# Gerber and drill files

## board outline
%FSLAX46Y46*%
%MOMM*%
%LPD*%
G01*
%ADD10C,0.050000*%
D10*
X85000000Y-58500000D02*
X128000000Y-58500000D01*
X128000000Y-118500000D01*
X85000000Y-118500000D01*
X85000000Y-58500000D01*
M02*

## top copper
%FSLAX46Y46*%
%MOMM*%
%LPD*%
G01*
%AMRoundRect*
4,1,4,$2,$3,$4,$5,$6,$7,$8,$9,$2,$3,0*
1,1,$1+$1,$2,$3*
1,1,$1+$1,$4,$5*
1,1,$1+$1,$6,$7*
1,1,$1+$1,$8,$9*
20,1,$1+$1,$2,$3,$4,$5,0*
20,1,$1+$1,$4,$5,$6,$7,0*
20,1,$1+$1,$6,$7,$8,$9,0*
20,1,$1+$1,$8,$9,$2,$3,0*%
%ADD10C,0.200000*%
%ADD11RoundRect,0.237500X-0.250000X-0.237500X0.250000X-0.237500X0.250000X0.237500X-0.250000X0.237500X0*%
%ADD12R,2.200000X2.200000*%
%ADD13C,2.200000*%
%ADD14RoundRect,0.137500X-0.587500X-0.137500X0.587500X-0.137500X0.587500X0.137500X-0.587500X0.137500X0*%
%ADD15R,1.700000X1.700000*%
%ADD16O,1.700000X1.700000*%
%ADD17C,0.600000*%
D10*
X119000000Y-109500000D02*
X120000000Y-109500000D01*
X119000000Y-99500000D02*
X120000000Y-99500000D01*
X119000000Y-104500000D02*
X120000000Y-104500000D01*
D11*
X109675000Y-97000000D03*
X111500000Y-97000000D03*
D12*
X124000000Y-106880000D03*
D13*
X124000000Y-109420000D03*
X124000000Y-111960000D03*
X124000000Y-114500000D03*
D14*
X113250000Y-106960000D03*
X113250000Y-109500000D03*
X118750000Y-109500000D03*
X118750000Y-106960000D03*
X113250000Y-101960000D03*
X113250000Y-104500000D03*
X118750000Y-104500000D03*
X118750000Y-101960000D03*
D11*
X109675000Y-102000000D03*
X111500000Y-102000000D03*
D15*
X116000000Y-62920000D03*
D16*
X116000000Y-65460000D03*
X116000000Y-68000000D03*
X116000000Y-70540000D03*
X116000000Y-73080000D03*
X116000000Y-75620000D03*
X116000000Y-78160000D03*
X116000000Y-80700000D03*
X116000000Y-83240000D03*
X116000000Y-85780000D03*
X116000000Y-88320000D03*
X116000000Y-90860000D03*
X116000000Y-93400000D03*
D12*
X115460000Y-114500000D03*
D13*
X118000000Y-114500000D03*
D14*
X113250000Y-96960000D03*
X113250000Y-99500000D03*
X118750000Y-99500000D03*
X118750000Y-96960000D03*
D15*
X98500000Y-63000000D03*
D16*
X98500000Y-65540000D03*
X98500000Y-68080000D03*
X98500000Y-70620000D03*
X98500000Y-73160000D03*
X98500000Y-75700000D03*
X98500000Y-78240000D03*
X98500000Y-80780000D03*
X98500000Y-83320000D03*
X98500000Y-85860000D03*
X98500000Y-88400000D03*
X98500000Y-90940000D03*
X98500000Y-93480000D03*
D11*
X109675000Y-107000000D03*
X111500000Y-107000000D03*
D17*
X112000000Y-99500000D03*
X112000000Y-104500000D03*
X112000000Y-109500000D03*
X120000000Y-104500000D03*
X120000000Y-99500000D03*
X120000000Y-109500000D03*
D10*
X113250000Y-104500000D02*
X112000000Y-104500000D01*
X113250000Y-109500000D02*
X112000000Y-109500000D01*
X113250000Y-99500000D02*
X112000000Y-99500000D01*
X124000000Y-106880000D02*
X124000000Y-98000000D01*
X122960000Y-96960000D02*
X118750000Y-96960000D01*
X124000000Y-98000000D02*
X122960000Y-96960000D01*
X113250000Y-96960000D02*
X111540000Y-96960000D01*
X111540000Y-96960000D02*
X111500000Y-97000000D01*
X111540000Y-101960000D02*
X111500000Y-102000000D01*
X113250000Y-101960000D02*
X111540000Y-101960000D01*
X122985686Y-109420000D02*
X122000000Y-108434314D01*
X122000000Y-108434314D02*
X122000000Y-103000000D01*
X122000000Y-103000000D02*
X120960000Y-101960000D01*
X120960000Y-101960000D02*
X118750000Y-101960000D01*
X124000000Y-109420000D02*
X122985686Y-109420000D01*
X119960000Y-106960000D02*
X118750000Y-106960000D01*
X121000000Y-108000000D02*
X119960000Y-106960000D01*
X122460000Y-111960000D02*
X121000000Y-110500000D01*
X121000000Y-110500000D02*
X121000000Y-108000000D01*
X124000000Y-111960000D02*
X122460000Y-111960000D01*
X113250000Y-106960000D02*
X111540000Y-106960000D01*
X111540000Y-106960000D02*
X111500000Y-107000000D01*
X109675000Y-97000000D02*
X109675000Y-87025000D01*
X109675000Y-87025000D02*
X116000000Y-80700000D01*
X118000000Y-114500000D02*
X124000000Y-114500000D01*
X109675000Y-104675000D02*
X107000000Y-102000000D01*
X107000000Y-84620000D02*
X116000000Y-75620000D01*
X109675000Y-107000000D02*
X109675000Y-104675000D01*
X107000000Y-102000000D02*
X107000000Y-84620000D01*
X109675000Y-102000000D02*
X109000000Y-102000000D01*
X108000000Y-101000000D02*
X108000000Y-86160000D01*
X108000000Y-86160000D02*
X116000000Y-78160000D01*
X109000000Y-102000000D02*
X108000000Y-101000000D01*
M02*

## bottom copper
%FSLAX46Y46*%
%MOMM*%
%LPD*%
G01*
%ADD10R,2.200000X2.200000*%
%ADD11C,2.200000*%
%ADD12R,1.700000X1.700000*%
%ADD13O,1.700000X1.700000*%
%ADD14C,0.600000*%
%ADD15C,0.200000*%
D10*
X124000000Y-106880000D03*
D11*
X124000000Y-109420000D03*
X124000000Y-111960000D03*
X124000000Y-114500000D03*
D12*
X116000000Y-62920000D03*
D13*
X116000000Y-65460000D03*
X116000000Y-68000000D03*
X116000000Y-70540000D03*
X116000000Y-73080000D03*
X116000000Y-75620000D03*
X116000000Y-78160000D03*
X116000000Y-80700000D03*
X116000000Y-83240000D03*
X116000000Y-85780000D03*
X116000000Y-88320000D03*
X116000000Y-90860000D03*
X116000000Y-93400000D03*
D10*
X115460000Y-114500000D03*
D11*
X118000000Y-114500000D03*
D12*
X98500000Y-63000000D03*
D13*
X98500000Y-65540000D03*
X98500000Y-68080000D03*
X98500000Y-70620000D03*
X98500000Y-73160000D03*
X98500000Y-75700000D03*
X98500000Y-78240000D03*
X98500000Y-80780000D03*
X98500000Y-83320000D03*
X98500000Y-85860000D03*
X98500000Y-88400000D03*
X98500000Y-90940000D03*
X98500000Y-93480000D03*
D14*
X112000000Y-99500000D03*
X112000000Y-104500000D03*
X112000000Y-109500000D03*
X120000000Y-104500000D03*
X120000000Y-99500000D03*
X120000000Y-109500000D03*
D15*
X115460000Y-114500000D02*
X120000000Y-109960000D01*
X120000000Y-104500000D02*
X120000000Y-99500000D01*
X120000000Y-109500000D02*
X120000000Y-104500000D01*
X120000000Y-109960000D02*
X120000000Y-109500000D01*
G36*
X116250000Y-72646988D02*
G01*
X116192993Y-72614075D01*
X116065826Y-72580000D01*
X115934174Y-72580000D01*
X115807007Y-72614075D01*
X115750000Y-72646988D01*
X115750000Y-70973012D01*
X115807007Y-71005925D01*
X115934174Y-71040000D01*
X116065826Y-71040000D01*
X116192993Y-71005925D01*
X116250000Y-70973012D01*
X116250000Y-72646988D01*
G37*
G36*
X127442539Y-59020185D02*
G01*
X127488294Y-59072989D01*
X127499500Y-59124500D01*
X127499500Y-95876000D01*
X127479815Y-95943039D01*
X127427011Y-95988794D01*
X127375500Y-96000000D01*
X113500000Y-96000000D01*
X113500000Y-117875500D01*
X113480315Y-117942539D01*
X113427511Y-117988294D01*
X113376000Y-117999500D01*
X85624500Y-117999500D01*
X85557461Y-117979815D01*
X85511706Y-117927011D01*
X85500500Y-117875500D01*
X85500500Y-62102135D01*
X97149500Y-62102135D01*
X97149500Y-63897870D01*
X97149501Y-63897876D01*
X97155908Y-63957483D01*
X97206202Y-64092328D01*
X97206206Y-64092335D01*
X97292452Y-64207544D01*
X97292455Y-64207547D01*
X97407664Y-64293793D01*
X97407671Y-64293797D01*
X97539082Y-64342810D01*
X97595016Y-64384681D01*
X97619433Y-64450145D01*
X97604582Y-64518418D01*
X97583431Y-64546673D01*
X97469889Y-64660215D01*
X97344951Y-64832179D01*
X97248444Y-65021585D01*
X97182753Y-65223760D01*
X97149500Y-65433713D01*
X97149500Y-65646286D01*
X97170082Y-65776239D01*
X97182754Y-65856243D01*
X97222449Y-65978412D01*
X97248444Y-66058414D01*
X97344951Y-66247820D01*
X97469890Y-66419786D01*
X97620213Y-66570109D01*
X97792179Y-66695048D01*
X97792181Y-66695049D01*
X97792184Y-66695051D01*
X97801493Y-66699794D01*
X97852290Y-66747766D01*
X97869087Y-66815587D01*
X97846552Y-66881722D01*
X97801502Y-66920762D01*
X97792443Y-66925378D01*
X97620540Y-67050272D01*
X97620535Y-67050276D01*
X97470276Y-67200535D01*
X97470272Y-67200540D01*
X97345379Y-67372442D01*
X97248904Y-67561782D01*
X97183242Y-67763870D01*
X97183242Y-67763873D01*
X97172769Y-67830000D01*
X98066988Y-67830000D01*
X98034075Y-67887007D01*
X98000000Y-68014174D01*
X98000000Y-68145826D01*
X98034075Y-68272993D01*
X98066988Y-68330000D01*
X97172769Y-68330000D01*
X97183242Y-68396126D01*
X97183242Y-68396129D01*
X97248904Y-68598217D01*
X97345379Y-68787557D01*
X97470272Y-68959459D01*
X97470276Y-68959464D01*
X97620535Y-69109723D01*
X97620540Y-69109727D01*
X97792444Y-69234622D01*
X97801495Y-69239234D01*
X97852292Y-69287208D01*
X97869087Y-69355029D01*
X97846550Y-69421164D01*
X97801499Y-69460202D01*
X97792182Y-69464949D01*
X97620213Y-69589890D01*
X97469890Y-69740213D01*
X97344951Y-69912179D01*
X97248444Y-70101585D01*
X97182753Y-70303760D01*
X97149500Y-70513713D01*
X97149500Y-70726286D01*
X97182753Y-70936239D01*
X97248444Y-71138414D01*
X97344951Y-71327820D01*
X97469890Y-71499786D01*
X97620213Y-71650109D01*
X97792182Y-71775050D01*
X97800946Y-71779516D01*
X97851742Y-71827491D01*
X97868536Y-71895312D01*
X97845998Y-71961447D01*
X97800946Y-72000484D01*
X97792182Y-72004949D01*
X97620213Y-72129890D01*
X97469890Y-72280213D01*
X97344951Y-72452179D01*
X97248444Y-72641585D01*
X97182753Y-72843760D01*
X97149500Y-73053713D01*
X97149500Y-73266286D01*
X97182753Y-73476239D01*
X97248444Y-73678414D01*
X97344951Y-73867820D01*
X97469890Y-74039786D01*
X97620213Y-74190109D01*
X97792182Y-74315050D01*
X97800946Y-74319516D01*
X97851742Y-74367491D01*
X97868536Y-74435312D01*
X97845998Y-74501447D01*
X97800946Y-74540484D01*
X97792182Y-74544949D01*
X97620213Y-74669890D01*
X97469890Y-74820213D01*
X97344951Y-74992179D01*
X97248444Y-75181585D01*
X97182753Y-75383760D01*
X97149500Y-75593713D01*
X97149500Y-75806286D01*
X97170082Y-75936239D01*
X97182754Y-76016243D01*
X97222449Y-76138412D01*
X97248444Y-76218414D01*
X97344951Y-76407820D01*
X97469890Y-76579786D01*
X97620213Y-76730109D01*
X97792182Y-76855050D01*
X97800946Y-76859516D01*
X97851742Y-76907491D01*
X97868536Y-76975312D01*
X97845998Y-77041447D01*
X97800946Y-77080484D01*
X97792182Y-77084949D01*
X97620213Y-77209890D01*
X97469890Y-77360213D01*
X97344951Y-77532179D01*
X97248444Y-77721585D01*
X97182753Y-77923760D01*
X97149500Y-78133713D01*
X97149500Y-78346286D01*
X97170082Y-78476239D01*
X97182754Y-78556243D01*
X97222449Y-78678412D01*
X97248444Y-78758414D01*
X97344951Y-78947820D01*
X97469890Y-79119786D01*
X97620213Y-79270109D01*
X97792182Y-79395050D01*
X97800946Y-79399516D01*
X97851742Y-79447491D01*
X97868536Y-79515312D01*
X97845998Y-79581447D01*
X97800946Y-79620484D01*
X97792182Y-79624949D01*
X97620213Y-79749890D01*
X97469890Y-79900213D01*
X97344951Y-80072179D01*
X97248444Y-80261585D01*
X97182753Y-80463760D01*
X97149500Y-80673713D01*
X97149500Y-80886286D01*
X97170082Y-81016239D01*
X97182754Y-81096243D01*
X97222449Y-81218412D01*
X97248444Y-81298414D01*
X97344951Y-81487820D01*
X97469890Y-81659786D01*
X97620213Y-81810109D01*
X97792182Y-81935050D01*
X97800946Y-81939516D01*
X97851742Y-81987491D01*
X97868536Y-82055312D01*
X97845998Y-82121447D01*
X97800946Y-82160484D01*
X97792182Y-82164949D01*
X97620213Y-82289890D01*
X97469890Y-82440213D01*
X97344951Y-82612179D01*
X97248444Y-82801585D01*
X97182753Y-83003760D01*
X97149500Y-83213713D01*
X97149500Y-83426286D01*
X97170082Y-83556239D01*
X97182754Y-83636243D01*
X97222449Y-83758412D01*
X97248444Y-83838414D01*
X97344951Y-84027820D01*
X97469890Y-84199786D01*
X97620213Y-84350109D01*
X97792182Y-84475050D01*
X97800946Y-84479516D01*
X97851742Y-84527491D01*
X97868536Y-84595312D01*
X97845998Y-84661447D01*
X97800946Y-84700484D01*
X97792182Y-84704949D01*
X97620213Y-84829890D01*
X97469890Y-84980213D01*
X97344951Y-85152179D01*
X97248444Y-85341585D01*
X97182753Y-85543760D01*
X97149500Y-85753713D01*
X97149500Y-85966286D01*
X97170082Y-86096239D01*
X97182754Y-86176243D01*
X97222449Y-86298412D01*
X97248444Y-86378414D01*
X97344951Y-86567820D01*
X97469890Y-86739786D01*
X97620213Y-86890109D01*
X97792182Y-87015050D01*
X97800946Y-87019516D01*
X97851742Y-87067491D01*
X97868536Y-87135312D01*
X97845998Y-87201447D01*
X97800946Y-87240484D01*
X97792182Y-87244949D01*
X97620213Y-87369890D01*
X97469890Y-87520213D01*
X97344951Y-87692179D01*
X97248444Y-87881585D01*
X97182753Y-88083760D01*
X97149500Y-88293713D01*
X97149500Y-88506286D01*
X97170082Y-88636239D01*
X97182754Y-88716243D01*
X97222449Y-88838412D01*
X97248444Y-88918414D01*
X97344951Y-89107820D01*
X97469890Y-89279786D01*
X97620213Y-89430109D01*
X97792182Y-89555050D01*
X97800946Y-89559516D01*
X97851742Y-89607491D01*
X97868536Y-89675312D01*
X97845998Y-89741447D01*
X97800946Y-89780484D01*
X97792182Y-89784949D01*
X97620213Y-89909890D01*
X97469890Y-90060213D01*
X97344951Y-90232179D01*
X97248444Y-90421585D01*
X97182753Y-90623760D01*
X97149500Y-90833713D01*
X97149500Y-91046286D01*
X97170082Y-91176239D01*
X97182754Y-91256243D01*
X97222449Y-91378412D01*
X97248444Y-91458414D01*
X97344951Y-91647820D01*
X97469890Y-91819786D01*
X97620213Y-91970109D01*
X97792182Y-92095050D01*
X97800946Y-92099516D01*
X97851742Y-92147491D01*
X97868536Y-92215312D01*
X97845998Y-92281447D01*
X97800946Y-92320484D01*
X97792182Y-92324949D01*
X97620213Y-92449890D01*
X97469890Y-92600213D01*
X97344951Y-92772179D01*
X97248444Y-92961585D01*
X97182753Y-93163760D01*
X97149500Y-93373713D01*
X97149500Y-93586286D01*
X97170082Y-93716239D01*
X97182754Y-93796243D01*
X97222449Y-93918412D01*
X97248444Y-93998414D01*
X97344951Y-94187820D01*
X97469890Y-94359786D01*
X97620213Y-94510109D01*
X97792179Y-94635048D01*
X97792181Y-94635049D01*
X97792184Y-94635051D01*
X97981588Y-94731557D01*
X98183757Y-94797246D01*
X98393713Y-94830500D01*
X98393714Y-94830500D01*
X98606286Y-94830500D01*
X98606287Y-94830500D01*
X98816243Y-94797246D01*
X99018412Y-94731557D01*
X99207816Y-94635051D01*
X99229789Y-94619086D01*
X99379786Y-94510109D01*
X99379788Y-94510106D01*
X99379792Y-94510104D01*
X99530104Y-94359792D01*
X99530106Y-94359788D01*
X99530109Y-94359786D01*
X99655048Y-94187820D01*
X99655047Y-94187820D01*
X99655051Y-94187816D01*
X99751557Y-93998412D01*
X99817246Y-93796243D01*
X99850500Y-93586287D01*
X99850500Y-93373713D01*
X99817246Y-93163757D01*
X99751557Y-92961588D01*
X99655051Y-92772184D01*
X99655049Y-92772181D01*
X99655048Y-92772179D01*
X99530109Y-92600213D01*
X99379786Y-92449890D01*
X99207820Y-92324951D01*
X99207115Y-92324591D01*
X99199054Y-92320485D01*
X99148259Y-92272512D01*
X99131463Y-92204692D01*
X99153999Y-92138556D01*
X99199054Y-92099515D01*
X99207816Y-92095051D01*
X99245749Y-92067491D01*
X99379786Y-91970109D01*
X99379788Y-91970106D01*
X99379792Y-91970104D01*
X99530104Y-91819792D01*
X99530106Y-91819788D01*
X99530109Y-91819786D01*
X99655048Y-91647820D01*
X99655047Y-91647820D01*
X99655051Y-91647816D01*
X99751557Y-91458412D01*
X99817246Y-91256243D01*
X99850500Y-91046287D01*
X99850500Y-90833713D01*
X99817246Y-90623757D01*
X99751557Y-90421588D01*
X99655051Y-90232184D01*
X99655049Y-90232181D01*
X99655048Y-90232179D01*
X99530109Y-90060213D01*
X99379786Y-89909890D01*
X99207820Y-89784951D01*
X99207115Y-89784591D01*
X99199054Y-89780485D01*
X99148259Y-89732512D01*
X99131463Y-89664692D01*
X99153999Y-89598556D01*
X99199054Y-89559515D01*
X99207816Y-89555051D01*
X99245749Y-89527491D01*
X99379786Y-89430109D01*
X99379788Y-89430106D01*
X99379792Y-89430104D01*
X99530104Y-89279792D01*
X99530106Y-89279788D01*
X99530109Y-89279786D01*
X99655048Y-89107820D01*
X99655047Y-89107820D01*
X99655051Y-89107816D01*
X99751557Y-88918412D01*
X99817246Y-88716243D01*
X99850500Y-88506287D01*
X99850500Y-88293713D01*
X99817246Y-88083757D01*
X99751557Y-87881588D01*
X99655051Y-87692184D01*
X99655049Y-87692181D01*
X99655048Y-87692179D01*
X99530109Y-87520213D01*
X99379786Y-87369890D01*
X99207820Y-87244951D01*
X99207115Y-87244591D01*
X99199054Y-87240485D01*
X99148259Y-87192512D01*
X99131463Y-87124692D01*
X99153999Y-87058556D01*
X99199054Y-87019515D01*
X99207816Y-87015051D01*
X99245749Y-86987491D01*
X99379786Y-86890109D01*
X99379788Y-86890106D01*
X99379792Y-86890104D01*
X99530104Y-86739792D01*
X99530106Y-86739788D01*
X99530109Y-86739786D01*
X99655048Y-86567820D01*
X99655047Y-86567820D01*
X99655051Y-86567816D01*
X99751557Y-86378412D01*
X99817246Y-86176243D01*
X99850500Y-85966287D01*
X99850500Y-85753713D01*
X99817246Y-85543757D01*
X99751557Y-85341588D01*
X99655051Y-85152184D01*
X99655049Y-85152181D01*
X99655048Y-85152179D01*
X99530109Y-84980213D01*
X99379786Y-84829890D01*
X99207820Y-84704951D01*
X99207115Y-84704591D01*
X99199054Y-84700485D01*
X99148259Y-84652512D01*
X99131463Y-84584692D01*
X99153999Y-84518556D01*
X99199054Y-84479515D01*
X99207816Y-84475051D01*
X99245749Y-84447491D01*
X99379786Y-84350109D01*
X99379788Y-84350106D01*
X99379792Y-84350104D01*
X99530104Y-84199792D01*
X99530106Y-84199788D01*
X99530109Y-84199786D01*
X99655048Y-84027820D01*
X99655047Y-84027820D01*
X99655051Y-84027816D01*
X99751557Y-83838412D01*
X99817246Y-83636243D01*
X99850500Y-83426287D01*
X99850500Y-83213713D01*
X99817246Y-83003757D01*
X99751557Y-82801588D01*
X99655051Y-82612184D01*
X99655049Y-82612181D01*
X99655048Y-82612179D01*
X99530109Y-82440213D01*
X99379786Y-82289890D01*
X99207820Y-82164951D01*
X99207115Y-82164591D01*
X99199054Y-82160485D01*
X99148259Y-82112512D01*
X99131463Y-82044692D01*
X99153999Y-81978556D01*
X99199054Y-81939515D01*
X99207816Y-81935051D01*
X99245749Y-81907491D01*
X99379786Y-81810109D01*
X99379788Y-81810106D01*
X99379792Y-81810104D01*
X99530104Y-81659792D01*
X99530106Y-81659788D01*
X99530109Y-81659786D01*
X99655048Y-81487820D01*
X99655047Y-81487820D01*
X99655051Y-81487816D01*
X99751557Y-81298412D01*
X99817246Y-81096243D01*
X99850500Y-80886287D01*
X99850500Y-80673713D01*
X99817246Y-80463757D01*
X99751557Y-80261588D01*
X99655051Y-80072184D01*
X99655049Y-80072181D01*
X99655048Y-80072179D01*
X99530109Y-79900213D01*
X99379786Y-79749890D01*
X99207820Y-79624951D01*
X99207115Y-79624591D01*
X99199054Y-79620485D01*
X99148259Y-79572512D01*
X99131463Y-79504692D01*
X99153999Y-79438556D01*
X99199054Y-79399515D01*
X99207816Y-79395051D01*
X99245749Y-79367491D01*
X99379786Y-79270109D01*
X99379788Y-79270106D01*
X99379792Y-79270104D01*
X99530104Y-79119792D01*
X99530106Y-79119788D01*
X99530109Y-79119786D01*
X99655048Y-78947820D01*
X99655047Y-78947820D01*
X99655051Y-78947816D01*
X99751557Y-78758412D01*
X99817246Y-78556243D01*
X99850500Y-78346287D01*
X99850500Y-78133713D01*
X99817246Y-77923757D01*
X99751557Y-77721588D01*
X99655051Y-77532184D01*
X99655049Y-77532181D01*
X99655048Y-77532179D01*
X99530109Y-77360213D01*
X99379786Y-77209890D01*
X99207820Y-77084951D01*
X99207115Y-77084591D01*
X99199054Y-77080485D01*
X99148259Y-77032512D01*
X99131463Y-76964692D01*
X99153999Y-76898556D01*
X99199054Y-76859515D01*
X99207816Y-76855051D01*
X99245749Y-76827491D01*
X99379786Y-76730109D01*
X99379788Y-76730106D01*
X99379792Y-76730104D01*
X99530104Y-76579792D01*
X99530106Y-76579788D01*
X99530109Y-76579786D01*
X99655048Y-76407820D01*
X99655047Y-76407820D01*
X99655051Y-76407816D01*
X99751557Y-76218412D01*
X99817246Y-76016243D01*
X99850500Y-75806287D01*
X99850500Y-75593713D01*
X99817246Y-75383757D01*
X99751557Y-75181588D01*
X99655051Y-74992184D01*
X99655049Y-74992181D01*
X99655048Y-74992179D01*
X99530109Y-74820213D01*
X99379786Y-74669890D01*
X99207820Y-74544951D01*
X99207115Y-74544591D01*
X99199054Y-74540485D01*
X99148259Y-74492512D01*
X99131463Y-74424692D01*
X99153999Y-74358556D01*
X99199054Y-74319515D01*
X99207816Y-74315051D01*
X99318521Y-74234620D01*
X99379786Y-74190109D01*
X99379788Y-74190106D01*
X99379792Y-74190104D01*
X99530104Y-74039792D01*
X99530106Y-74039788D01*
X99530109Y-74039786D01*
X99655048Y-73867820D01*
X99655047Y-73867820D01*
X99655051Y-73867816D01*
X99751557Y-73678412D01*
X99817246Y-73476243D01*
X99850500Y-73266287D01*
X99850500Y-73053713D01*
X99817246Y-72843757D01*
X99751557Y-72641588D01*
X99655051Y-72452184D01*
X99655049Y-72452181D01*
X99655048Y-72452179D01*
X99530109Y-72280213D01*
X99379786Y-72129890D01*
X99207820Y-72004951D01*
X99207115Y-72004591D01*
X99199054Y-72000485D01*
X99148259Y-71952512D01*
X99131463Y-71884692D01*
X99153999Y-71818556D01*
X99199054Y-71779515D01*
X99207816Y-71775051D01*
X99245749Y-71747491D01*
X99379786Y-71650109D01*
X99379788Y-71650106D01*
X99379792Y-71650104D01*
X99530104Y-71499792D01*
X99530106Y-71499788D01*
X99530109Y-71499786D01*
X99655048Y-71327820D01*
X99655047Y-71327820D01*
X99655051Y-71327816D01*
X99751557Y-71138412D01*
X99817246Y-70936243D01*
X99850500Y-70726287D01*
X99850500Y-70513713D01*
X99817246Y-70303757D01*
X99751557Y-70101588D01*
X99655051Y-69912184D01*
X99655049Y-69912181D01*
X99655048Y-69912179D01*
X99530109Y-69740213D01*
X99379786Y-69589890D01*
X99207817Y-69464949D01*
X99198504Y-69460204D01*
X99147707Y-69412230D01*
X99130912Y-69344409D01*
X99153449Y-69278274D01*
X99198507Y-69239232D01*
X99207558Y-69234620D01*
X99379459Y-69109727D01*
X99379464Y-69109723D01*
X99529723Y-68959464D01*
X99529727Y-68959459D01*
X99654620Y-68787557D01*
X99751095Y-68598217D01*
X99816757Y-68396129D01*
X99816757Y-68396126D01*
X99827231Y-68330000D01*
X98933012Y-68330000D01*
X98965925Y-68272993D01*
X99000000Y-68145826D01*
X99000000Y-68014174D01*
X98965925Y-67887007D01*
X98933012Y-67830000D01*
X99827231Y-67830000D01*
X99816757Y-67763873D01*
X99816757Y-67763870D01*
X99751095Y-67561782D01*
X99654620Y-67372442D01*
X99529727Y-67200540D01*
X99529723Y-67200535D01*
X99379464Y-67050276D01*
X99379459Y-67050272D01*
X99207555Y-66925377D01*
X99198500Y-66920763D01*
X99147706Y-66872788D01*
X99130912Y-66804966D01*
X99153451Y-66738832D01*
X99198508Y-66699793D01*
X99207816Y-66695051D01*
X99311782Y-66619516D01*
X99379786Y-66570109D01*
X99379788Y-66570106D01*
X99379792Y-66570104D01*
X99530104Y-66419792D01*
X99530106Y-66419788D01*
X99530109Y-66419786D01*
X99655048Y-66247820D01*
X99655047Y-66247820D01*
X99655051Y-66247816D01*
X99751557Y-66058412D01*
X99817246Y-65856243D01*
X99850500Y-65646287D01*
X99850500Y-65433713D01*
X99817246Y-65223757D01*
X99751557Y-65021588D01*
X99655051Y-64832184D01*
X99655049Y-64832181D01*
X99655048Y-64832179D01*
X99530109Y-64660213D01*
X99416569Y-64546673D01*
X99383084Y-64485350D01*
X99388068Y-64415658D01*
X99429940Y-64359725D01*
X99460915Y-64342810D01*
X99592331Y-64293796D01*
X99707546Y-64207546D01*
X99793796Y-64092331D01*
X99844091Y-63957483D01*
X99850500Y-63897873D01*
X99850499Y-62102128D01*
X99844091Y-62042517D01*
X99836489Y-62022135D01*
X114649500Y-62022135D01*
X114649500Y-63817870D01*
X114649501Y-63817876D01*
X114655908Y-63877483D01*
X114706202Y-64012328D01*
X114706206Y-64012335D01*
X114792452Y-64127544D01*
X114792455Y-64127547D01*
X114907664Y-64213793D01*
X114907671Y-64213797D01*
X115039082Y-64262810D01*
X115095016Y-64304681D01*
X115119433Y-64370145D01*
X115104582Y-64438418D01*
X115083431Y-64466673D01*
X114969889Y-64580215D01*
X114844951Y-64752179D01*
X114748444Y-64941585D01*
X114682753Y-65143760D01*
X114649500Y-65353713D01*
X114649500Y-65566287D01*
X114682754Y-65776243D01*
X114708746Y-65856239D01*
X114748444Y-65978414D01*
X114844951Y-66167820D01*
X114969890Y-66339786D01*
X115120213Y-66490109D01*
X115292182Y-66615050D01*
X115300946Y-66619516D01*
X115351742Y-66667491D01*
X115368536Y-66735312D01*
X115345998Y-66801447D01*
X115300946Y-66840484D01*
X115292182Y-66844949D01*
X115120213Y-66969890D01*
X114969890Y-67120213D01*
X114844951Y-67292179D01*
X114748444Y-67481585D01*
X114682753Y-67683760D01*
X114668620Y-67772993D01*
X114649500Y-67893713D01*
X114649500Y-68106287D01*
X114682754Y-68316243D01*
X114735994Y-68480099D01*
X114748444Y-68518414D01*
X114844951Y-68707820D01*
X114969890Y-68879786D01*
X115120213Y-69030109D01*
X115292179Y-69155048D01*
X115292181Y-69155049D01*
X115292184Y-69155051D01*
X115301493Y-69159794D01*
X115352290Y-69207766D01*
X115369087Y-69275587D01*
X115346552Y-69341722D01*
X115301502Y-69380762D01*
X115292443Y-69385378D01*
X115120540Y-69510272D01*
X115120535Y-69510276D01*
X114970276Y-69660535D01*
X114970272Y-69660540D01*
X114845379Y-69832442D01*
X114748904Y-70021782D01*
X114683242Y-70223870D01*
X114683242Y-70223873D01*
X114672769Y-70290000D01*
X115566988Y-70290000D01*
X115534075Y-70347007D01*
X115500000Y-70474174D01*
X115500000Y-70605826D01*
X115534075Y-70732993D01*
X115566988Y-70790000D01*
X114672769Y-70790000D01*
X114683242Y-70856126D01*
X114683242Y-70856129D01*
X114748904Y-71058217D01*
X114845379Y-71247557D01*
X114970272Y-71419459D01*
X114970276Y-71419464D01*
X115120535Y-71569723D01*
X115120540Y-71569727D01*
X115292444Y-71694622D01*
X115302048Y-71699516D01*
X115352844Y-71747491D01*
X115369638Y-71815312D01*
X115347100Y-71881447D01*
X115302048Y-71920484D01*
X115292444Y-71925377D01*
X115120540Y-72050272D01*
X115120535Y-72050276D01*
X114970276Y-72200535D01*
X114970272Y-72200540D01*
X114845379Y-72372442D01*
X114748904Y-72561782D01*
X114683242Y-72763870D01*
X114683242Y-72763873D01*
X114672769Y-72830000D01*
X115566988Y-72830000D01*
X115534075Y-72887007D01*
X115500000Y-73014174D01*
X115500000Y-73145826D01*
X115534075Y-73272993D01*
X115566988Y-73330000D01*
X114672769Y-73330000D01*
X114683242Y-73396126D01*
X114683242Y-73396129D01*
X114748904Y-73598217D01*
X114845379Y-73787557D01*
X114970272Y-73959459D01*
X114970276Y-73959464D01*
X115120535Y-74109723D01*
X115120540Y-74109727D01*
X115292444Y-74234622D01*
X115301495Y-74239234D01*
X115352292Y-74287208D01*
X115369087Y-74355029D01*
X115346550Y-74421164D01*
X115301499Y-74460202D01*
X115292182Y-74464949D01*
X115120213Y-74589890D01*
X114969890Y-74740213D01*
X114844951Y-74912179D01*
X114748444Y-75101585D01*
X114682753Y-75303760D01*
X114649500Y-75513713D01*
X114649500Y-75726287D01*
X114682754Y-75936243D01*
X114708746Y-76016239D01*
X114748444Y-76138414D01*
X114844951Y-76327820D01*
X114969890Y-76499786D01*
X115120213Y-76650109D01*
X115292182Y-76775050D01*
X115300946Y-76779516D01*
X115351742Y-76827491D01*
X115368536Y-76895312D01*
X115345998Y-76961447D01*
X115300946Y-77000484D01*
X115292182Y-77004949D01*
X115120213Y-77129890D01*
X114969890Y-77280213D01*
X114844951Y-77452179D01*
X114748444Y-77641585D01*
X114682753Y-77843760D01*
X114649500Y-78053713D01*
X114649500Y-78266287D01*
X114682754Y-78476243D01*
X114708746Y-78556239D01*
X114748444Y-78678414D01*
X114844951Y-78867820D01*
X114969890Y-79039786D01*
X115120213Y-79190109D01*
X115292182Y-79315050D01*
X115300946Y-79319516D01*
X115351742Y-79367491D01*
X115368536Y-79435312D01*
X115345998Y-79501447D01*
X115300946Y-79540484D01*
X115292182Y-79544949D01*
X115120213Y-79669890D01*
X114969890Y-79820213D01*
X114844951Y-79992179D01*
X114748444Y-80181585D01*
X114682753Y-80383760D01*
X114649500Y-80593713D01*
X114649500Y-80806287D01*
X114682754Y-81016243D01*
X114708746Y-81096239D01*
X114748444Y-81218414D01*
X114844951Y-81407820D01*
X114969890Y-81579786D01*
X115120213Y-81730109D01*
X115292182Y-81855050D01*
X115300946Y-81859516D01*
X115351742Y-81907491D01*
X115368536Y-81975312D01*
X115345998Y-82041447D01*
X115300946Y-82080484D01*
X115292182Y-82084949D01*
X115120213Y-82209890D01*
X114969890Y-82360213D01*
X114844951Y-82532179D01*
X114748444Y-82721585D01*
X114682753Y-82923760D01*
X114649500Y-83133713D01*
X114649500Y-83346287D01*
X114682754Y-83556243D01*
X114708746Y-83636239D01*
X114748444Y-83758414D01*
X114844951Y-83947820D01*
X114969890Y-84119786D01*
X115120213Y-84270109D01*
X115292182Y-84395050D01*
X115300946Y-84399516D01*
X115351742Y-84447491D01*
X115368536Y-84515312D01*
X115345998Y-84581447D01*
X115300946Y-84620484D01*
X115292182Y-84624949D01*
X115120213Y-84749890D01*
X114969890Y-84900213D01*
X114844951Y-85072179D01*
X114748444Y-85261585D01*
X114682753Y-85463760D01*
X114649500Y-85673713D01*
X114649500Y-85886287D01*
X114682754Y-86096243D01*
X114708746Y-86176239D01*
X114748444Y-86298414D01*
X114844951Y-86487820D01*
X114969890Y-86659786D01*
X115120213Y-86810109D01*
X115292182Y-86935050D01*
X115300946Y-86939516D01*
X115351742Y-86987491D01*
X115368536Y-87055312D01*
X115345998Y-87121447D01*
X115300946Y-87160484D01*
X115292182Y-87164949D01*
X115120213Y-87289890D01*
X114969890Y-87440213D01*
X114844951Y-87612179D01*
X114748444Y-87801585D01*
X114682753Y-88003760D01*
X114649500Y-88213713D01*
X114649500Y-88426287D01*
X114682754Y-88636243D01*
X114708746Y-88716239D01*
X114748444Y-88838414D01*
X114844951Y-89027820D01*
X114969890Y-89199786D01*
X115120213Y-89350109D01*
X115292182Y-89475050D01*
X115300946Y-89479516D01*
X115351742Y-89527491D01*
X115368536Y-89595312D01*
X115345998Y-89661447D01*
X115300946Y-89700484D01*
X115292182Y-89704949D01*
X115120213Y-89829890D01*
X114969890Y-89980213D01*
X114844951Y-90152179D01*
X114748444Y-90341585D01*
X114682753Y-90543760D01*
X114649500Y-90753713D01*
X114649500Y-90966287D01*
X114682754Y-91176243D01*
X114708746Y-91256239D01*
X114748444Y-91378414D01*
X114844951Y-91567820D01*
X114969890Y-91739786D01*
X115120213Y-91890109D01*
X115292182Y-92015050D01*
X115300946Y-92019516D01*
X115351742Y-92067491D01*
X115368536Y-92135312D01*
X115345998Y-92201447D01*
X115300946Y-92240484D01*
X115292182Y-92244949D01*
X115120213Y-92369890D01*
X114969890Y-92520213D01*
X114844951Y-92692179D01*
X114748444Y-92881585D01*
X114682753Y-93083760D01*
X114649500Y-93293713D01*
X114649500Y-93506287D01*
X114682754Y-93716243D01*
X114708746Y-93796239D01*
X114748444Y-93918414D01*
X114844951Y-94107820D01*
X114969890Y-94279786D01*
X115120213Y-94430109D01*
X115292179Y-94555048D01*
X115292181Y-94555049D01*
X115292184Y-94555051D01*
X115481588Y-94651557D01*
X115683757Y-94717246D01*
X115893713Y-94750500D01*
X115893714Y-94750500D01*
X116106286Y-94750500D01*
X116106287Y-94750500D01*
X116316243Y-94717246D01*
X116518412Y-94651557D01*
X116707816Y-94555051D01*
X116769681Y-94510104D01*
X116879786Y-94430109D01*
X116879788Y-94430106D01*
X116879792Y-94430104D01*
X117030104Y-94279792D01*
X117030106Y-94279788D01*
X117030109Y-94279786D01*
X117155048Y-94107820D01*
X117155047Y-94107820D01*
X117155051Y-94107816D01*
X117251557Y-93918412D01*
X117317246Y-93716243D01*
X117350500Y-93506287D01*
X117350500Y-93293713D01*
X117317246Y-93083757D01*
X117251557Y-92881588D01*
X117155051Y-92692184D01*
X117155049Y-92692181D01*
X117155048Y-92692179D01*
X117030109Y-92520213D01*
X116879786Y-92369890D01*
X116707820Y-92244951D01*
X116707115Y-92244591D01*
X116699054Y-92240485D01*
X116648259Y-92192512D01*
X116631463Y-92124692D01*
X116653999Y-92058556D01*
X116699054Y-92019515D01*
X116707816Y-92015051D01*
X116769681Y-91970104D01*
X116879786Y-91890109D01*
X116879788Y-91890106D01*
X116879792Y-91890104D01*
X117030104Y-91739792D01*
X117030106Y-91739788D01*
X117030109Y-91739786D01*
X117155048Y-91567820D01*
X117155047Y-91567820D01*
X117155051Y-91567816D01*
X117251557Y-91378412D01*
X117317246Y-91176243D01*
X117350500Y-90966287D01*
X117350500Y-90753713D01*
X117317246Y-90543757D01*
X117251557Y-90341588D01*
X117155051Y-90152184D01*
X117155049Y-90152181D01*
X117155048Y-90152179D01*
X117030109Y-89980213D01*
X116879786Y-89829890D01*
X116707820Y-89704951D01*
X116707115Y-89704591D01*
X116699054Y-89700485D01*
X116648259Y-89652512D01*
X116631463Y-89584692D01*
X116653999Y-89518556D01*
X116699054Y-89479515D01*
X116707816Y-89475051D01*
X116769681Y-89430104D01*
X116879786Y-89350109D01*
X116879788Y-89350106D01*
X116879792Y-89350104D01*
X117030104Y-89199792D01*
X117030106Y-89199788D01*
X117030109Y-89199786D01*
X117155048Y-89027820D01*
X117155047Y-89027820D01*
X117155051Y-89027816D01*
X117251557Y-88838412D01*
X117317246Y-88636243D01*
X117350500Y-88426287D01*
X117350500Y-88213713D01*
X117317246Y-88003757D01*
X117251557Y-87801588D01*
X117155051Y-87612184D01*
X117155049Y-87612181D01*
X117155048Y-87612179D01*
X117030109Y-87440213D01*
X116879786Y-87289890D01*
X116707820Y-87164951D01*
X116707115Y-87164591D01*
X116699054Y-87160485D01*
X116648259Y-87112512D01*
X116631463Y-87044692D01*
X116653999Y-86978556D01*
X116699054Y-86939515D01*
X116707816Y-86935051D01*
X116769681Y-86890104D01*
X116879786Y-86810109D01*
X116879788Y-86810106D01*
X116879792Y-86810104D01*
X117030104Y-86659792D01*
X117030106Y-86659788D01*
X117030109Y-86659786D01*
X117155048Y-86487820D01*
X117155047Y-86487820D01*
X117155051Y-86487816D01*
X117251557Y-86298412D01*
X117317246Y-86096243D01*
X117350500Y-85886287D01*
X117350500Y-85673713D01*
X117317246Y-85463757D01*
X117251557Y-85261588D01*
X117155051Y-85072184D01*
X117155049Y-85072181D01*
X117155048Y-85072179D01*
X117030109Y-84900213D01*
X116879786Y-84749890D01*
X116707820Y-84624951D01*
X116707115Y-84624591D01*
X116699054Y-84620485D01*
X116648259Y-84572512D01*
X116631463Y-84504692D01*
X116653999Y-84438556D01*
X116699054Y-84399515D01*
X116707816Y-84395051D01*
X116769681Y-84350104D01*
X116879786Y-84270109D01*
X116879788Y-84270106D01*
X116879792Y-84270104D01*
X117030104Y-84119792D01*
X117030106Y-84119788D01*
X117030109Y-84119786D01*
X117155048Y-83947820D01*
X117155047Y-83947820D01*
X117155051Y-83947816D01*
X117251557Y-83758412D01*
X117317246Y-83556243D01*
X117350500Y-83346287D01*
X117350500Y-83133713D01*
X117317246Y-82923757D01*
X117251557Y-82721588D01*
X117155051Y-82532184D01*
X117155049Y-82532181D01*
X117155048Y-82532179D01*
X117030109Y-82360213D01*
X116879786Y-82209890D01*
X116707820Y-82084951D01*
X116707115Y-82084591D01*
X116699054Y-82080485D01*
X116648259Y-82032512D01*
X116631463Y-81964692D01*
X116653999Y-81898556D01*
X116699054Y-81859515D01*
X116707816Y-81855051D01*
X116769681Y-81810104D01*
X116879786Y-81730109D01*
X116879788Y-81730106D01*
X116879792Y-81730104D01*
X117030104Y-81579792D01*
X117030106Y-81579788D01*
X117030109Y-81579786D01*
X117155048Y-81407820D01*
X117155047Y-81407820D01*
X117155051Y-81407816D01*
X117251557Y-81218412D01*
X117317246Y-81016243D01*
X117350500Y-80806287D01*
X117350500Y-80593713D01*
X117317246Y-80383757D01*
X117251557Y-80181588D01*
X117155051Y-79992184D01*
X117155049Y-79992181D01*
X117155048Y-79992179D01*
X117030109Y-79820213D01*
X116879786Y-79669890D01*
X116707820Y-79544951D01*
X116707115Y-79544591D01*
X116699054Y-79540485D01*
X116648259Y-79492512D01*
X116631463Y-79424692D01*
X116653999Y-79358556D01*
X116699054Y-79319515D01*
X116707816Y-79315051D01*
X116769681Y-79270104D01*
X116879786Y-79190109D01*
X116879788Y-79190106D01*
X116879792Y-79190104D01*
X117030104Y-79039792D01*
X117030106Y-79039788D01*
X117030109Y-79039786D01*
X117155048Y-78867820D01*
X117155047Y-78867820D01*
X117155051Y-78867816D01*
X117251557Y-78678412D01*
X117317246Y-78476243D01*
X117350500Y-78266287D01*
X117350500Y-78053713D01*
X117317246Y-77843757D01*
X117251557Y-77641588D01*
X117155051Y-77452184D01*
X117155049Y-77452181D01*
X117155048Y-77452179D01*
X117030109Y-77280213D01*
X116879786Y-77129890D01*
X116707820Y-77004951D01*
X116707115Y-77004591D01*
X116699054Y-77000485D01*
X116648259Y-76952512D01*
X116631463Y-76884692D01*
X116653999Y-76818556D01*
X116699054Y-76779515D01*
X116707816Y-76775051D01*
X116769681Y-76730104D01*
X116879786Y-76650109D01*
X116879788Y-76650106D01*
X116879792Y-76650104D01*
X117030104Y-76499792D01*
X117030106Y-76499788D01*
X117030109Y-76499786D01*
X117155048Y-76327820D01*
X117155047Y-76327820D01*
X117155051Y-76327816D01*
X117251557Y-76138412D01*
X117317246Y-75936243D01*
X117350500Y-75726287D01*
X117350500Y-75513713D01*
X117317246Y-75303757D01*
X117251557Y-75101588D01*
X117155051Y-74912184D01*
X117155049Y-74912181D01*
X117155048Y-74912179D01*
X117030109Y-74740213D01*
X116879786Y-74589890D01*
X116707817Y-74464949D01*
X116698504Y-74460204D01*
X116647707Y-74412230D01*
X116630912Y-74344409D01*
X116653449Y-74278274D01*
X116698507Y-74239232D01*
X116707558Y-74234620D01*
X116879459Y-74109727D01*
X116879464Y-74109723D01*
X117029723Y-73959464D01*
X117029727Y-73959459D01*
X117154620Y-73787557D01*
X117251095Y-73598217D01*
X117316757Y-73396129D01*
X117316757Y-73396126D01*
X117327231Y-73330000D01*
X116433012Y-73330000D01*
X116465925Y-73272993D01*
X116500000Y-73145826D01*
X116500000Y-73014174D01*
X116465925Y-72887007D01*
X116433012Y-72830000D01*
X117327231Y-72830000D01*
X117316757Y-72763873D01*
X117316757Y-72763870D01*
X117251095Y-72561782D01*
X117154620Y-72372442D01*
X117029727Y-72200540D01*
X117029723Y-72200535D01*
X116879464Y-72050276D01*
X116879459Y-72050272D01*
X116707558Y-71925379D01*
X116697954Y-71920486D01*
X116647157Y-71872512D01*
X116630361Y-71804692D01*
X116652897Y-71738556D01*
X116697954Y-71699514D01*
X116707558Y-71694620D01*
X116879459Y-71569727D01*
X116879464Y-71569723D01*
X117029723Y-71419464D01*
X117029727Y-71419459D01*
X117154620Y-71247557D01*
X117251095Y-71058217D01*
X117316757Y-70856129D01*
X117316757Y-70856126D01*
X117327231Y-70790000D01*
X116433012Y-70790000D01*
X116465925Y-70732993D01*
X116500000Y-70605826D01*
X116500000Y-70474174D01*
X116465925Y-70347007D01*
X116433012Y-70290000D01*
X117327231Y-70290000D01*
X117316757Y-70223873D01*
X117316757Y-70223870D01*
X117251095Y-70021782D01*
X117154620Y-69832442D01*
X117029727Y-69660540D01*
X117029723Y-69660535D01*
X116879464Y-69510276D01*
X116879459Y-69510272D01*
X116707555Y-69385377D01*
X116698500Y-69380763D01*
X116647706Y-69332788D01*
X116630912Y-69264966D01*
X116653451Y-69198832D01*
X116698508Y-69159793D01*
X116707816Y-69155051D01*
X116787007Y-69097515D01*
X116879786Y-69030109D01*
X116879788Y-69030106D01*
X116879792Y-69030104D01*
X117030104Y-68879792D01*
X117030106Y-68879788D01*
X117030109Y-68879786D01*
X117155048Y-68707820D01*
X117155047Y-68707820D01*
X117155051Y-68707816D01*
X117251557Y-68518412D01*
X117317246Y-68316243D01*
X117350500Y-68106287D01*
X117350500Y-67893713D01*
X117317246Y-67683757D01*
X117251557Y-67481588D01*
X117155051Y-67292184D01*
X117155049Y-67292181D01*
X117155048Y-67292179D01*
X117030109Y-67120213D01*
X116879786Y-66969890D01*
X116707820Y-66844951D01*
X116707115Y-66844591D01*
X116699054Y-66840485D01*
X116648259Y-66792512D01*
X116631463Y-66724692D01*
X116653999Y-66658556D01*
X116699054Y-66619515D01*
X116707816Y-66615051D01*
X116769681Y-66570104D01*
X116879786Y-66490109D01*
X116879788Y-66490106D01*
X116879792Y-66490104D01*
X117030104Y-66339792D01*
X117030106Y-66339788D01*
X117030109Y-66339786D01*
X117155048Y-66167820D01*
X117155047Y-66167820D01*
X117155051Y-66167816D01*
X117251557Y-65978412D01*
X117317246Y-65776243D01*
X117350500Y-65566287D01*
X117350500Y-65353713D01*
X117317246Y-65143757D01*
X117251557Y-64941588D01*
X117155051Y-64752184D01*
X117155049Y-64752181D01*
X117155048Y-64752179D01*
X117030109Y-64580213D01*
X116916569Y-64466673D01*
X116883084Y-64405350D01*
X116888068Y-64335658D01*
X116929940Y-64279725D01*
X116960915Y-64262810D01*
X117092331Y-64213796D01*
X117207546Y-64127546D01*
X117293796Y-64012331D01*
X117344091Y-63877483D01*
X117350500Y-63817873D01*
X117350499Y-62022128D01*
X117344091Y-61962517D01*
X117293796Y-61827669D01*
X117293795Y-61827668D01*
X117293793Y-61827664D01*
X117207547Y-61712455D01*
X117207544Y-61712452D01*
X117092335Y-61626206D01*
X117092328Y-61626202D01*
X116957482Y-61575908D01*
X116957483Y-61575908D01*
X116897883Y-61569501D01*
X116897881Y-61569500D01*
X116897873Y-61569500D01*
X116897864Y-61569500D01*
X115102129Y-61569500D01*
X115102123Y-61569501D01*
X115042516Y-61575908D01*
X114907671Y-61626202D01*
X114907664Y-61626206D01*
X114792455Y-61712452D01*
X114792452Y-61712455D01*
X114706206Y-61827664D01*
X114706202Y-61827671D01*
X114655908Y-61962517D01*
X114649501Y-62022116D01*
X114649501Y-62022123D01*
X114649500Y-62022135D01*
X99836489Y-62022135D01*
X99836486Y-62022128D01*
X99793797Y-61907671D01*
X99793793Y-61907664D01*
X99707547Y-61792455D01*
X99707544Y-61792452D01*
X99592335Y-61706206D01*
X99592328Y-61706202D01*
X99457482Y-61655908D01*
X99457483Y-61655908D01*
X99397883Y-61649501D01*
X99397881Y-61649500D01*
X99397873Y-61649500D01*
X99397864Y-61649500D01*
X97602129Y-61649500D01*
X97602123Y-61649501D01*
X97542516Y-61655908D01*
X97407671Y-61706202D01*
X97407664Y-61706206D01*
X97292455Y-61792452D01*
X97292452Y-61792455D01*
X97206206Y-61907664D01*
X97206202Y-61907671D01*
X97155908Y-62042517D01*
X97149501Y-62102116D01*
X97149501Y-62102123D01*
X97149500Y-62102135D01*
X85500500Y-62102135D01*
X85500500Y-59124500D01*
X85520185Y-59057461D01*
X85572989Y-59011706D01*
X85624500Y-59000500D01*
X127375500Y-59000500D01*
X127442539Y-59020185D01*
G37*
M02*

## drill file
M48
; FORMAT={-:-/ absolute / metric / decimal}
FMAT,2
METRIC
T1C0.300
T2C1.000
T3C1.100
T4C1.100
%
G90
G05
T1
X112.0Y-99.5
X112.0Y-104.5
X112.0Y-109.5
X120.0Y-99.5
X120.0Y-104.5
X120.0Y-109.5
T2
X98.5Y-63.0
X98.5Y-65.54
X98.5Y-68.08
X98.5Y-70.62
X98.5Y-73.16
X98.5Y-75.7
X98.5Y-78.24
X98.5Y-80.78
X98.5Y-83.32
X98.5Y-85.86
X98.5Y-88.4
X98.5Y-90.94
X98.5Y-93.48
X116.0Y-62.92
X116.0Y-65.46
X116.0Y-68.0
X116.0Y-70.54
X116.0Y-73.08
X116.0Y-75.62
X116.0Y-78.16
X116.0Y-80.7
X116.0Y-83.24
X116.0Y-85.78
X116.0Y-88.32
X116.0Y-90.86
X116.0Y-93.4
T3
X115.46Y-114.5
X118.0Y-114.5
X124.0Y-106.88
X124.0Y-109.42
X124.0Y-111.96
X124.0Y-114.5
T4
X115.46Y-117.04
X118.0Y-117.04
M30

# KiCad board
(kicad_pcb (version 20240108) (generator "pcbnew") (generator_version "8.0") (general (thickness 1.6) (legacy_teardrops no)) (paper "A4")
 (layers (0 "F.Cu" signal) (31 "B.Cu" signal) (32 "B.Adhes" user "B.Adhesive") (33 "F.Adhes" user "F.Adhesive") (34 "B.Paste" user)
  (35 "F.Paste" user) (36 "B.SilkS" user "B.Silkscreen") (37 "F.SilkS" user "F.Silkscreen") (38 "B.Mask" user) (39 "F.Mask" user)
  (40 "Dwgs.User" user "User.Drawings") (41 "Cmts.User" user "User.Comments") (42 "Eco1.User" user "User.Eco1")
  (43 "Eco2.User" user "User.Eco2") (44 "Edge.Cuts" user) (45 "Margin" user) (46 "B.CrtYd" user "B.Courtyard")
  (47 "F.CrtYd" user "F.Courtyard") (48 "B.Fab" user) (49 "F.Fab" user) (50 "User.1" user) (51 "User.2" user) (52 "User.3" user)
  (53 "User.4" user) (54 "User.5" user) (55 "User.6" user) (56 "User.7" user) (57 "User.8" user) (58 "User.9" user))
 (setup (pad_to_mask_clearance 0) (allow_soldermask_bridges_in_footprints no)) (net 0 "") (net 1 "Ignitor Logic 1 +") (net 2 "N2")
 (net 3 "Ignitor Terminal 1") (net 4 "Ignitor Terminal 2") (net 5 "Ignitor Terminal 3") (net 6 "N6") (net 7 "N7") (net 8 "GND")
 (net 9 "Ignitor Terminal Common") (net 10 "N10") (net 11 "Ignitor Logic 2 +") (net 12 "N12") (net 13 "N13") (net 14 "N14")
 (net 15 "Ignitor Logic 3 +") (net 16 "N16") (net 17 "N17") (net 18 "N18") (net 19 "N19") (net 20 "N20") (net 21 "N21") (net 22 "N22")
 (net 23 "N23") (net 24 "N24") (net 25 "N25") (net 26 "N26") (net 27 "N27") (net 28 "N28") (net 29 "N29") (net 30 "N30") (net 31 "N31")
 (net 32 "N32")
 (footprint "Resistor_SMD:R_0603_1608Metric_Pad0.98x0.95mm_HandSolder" (layer "F.Cu") (at 110.5875 97)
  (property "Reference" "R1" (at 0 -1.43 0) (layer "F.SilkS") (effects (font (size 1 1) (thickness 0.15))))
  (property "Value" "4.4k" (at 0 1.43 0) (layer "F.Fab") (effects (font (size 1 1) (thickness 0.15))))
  (pad "1" smd roundrect (at -0.9125 0) (size 0.975 0.95) (layers "F.Cu" "F.Paste" "F.Mask") (roundrect_rratio 0.25)
   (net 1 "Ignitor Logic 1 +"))
  (pad "2" smd roundrect (at 0.9125 0) (size 0.975 0.95) (layers "F.Cu" "F.Paste" "F.Mask") (roundrect_rratio 0.25) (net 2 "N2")))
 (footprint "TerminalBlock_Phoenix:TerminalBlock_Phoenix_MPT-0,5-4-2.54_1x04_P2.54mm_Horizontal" (layer "F.Cu") (at 124 106.88 -90)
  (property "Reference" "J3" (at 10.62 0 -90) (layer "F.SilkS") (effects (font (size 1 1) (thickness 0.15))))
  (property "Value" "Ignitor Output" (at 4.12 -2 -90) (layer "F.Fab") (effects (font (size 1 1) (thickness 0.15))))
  (pad "1" thru_hole rect (at 0 0 270) (size 2.2 2.2) (drill 1.1) (layers "*.Cu" "*.Mask") (remove_unused_layers no)
   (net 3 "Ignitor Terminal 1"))
  (pad "2" thru_hole circle (at 2.54 0 270) (size 2.2 2.2) (drill 1.1) (layers "*.Cu" "*.Mask") (remove_unused_layers no)
   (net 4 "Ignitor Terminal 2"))
  (pad "3" thru_hole circle (at 5.08 0 270) (size 2.2 2.2) (drill 1.1) (layers "*.Cu" "*.Mask") (remove_unused_layers no)
   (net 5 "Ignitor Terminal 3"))
  (pad "4" thru_hole circle (at 7.62 0 270) (size 2.2 2.2) (drill 1.1) (layers "*.Cu" "*.Mask") (remove_unused_layers no) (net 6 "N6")))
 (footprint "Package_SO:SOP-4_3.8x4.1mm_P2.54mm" (layer "F.Cu") (at 116 108.23)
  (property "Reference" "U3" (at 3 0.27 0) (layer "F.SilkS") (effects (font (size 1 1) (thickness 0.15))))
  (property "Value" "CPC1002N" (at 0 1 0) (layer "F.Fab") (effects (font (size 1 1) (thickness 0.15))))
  (pad "1" smd roundrect (at -2.75 -1.27) (size 1.45 0.55) (layers "F.Cu" "F.Paste" "F.Mask") (roundrect_rratio 0.25) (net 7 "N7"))
  (pad "2" smd roundrect (at -2.75 1.27) (size 1.45 0.55) (layers "F.Cu" "F.Paste" "F.Mask") (roundrect_rratio 0.25) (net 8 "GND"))
  (pad "3" smd roundrect (at 2.75 1.27) (size 1.45 0.55) (layers "F.Cu" "F.Paste" "F.Mask") (roundrect_rratio 0.25)
   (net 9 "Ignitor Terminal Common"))
  (pad "4" smd roundrect (at 2.75 -1.27) (size 1.45 0.55) (layers "F.Cu" "F.Paste" "F.Mask") (roundrect_rratio 0.25)
   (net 5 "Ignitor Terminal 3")))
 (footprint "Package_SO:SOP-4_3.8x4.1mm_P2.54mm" (layer "F.Cu") (at 116 103.23)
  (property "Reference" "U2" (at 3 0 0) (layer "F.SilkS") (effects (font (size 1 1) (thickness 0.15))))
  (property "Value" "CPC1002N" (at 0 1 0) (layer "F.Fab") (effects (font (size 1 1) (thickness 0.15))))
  (pad "1" smd roundrect (at -2.75 -1.27) (size 1.45 0.55) (layers "F.Cu" "F.Paste" "F.Mask") (roundrect_rratio 0.25) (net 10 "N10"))
  (pad "2" smd roundrect (at -2.75 1.27) (size 1.45 0.55) (layers "F.Cu" "F.Paste" "F.Mask") (roundrect_rratio 0.25) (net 8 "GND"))
  (pad "3" smd roundrect (at 2.75 1.27) (size 1.45 0.55) (layers "F.Cu" "F.Paste" "F.Mask") (roundrect_rratio 0.25)
   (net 9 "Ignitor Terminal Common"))
  (pad "4" smd roundrect (at 2.75 -1.27) (size 1.45 0.55) (layers "F.Cu" "F.Paste" "F.Mask") (roundrect_rratio 0.25)
   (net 4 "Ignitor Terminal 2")))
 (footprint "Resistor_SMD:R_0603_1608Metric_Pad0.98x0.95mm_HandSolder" (layer "F.Cu") (at 110.5875 102)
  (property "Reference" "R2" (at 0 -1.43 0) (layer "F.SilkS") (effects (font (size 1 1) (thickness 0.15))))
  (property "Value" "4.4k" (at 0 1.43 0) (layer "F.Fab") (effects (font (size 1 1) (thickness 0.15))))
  (pad "1" smd roundrect (at -0.9125 0) (size 0.975 0.95) (layers "F.Cu" "F.Paste" "F.Mask") (roundrect_rratio 0.25)
   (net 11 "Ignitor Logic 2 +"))
  (pad "2" smd roundrect (at 0.9125 0) (size 0.975 0.95) (layers "F.Cu" "F.Paste" "F.Mask") (roundrect_rratio 0.25) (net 10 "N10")))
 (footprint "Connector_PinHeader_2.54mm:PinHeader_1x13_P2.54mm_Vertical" (layer "F.Cu") (at 116 62.92)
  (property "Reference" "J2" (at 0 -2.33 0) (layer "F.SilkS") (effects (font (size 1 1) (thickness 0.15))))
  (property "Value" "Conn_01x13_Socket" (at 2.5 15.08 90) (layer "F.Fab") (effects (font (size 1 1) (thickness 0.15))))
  (pad "1" thru_hole rect (at 0 0) (size 1.7 1.7) (drill 1) (layers "*.Cu" "*.Mask") (remove_unused_layers no) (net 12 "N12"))
  (pad "2" thru_hole oval (at 0 2.54) (size 1.7 1.7) (drill 1) (layers "*.Cu" "*.Mask") (remove_unused_layers no) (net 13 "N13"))
  (pad "3" thru_hole oval (at 0 5.08) (size 1.7 1.7) (drill 1) (layers "*.Cu" "*.Mask") (remove_unused_layers no) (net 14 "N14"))
  (pad "4" thru_hole oval (at 0 7.62) (size 1.7 1.7) (drill 1) (layers "*.Cu" "*.Mask") (remove_unused_layers no) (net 8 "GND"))
  (pad "5" thru_hole oval (at 0 10.16) (size 1.7 1.7) (drill 1) (layers "*.Cu" "*.Mask") (remove_unused_layers no) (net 8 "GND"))
  (pad "6" thru_hole oval (at 0 12.7) (size 1.7 1.7) (drill 1) (layers "*.Cu" "*.Mask") (remove_unused_layers no)
   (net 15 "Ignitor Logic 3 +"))
  (pad "7" thru_hole oval (at 0 15.24) (size 1.7 1.7) (drill 1) (layers "*.Cu" "*.Mask") (remove_unused_layers no)
   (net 11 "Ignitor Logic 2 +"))
  (pad "8" thru_hole oval (at 0 17.78) (size 1.7 1.7) (drill 1) (layers "*.Cu" "*.Mask") (remove_unused_layers no)
   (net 1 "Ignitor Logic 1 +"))
  (pad "9" thru_hole oval (at 0 20.32) (size 1.7 1.7) (drill 1) (layers "*.Cu" "*.Mask") (remove_unused_layers no) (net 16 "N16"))
  (pad "10" thru_hole oval (at 0 22.86) (size 1.7 1.7) (drill 1) (layers "*.Cu" "*.Mask") (remove_unused_layers no) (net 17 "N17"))
  (pad "11" thru_hole oval (at 0 25.4) (size 1.7 1.7) (drill 1) (layers "*.Cu" "*.Mask") (remove_unused_layers no) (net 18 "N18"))
  (pad "12" thru_hole oval (at 0 27.94) (size 1.7 1.7) (drill 1) (layers "*.Cu" "*.Mask") (remove_unused_layers no) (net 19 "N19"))
  (pad "13" thru_hole oval (at 0 30.48) (size 1.7 1.7) (drill 1) (layers "*.Cu" "*.Mask") (remove_unused_layers no) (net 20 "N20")))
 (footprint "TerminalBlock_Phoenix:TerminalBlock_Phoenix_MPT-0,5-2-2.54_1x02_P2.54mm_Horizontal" (layer "F.Cu") (at 115.46 114.5)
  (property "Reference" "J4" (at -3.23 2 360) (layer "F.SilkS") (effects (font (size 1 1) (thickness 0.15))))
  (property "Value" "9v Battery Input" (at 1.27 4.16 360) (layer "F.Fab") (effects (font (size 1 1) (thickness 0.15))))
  (pad "" np_thru_hole circle (at 0 2.54) (size 1.1 1.1) (drill 1.1) (layers "*.Cu" "*.Mask"))
  (pad "" np_thru_hole circle (at 2.54 2.54) (size 1.1 1.1) (drill 1.1) (layers "*.Cu" "*.Mask"))
  (pad "1" thru_hole rect (at 0 0) (size 2.2 2.2) (drill 1.1) (layers "*.Cu" "*.Mask") (remove_unused_layers no)
   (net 9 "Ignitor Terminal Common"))
  (pad "2" thru_hole circle (at 2.54 0) (size 2.2 2.2) (drill 1.1) (layers "*.Cu" "*.Mask") (remove_unused_layers no) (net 6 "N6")))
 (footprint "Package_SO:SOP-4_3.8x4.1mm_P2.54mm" (layer "F.Cu") (at 116 98.23)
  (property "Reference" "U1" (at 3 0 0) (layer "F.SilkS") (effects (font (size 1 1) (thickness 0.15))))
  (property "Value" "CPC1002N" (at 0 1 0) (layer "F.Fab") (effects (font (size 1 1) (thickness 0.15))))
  (pad "1" smd roundrect (at -2.75 -1.27) (size 1.45 0.55) (layers "F.Cu" "F.Paste" "F.Mask") (roundrect_rratio 0.25) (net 2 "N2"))
  (pad "2" smd roundrect (at -2.75 1.27) (size 1.45 0.55) (layers "F.Cu" "F.Paste" "F.Mask") (roundrect_rratio 0.25) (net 8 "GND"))
  (pad "3" smd roundrect (at 2.75 1.27) (size 1.45 0.55) (layers "F.Cu" "F.Paste" "F.Mask") (roundrect_rratio 0.25)
   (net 9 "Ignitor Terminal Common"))
  (pad "4" smd roundrect (at 2.75 -1.27) (size 1.45 0.55) (layers "F.Cu" "F.Paste" "F.Mask") (roundrect_rratio 0.25)
   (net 3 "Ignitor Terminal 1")))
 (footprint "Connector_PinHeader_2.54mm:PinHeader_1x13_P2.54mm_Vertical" (layer "F.Cu") (at 98.5 63)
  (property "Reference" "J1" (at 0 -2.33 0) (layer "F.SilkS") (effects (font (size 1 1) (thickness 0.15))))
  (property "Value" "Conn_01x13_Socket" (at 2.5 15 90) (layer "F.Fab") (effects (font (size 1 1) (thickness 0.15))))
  (pad "1" thru_hole rect (at 0 0) (size 1.7 1.7) (drill 1) (layers "*.Cu" "*.Mask") (remove_unused_layers no) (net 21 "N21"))
  (pad "2" thru_hole oval (at 0 2.54) (size 1.7 1.7) (drill 1) (layers "*.Cu" "*.Mask") (remove_unused_layers no) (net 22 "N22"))
  (pad "3" thru_hole oval (at 0 5.08) (size 1.7 1.7) (drill 1) (layers "*.Cu" "*.Mask") (remove_unused_layers no) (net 8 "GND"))
  (pad "4" thru_hole oval (at 0 7.62) (size 1.7 1.7) (drill 1) (layers "*.Cu" "*.Mask") (remove_unused_layers no) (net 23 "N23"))
  (pad "5" thru_hole oval (at 0 10.16) (size 1.7 1.7) (drill 1) (layers "*.Cu" "*.Mask") (remove_unused_layers no) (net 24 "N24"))
  (pad "6" thru_hole oval (at 0 12.7) (size 1.7 1.7) (drill 1) (layers "*.Cu" "*.Mask") (remove_unused_layers no) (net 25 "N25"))
  (pad "7" thru_hole oval (at 0 15.24) (size 1.7 1.7) (drill 1) (layers "*.Cu" "*.Mask") (remove_unused_layers no) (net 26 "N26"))
  (pad "8" thru_hole oval (at 0 17.78) (size 1.7 1.7) (drill 1) (layers "*.Cu" "*.Mask") (remove_unused_layers no) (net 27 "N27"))
  (pad "9" thru_hole oval (at 0 20.32) (size 1.7 1.7) (drill 1) (layers "*.Cu" "*.Mask") (remove_unused_layers no) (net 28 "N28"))
  (pad "10" thru_hole oval (at 0 22.86) (size 1.7 1.7) (drill 1) (layers "*.Cu" "*.Mask") (remove_unused_layers no) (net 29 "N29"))
  (pad "11" thru_hole oval (at 0 25.4) (size 1.7 1.7) (drill 1) (layers "*.Cu" "*.Mask") (remove_unused_layers no) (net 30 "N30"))
  (pad "12" thru_hole oval (at 0 27.94) (size 1.7 1.7) (drill 1) (layers "*.Cu" "*.Mask") (remove_unused_layers no) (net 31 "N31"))
  (pad "13" thru_hole oval (at 0 30.48) (size 1.7 1.7) (drill 1) (layers "*.Cu" "*.Mask") (remove_unused_layers no) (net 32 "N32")))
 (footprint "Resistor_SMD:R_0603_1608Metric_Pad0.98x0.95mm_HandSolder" (layer "F.Cu") (at 110.5875 107)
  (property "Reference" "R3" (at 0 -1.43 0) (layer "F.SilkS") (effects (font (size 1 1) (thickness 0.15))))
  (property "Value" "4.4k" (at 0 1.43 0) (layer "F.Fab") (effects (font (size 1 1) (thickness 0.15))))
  (pad "1" smd roundrect (at -0.9125 0) (size 0.975 0.95) (layers "F.Cu" "F.Paste" "F.Mask") (roundrect_rratio 0.25)
   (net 15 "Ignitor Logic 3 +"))
  (pad "2" smd roundrect (at 0.9125 0) (size 0.975 0.95) (layers "F.Cu" "F.Paste" "F.Mask") (roundrect_rratio 0.25) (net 7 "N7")))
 (gr_line (start 119 109.5) (end 120 109.5) (stroke (width 0.2) (type default)) (layer "F.Cu") (net 9))
 (gr_line (start 119 99.5) (end 120 99.5) (stroke (width 0.2) (type default)) (layer "F.Cu") (net 9))
 (gr_line (start 119 104.5) (end 120 104.5) (stroke (width 0.2) (type default)) (layer "F.Cu") (net 9))
 (gr_rect (start 85 58.5) (end 128 118.5) (stroke (width 0.05) (type default)) (fill none) (layer "Edge.Cuts"))
 (segment (start 113.25 104.5) (end 112 104.5) (width 0.2) (layer "F.Cu") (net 8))
 (segment (start 113.25 109.5) (end 112 109.5) (width 0.2) (layer "F.Cu") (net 8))
 (segment (start 113.25 99.5) (end 112 99.5) (width 0.2) (layer "F.Cu") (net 8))
 (via (at 112 99.5) (size 0.6) (drill 0.3) (layers "F.Cu" "B.Cu") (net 8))
 (via (at 112 104.5) (size 0.6) (drill 0.3) (layers "F.Cu" "B.Cu") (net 8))
 (via (at 112 109.5) (size 0.6) (drill 0.3) (layers "F.Cu" "B.Cu") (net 8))
 (segment (start 124 106.88) (end 124 98) (width 0.2) (layer "F.Cu") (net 3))
 (segment (start 122.96 96.96) (end 118.75 96.96) (width 0.2) (layer "F.Cu") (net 3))
 (segment (start 124 98) (end 122.96 96.96) (width 0.2) (layer "F.Cu") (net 3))
 (segment (start 113.25 96.96) (end 111.54 96.96) (width 0.2) (layer "F.Cu") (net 2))
 (segment (start 111.54 96.96) (end 111.5 97) (width 0.2) (layer "F.Cu") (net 2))
 (via (at 120 104.5) (size 0.6) (drill 0.3) (layers "F.Cu" "B.Cu") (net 9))
 (via (at 120 99.5) (size 0.6) (drill 0.3) (layers "F.Cu" "B.Cu") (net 9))
 (via (at 120 109.5) (size 0.6) (drill 0.3) (layers "F.Cu" "B.Cu") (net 9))
 (segment (start 115.46 114.5) (end 120 109.96) (width 0.2) (layer "B.Cu") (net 9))
 (segment (start 120 104.5) (end 120 99.5) (width 0.2) (layer "B.Cu") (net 9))
 (segment (start 120 109.5) (end 120 104.5) (width 0.2) (layer "B.Cu") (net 9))
 (segment (start 120 109.96) (end 120 109.5) (width 0.2) (layer "B.Cu") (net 9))
 (segment (start 111.54 101.96) (end 111.5 102) (width 0.2) (layer "F.Cu") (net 10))
 (segment (start 113.25 101.96) (end 111.54 101.96) (width 0.2) (layer "F.Cu") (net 10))
 (segment (start 122.985686 109.42) (end 122 108.434314) (width 0.2) (layer "F.Cu") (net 4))
 (segment (start 122 108.434314) (end 122 103) (width 0.2) (layer "F.Cu") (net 4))
 (segment (start 122 103) (end 120.96 101.96) (width 0.2) (layer "F.Cu") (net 4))
 (segment (start 120.96 101.96) (end 118.75 101.96) (width 0.2) (layer "F.Cu") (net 4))
 (segment (start 124 109.42) (end 122.985686 109.42) (width 0.2) (layer "F.Cu") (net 4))
 (segment (start 119.96 106.96) (end 118.75 106.96) (width 0.2) (layer "F.Cu") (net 5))
 (segment (start 121 108) (end 119.96 106.96) (width 0.2) (layer "F.Cu") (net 5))
 (segment (start 122.46 111.96) (end 121 110.5) (width 0.2) (layer "F.Cu") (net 5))
 (segment (start 121 110.5) (end 121 108) (width 0.2) (layer "F.Cu") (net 5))
 (segment (start 124 111.96) (end 122.46 111.96) (width 0.2) (layer "F.Cu") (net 5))
 (segment (start 113.25 106.96) (end 111.54 106.96) (width 0.2) (layer "F.Cu") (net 7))
 (segment (start 111.54 106.96) (end 111.5 107) (width 0.2) (layer "F.Cu") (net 7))
 (segment (start 109.675 97) (end 109.675 87.025) (width 0.2) (layer "F.Cu") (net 1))
 (segment (start 109.675 87.025) (end 116 80.7) (width 0.2) (layer "F.Cu") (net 1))
 (segment (start 118 114.5) (end 124 114.5) (width 0.2) (layer "F.Cu") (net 6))
 (segment (start 109.675 104.675) (end 107 102) (width 0.2) (layer "F.Cu") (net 15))
 (segment (start 107 84.62) (end 116 75.62) (width 0.2) (layer "F.Cu") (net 15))
 (segment (start 109.675 107) (end 109.675 104.675) (width 0.2) (layer "F.Cu") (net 15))
 (segment (start 107 102) (end 107 84.62) (width 0.2) (layer "F.Cu") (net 15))
 (segment (start 109.675 102) (end 109 102) (width 0.2) (layer "F.Cu") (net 11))
 (segment (start 108 101) (end 108 86.16) (width 0.2) (layer "F.Cu") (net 11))
 (segment (start 108 86.16) (end 116 78.16) (width 0.2) (layer "F.Cu") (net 11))
 (segment (start 109 102) (end 108 101) (width 0.2) (layer "F.Cu") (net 11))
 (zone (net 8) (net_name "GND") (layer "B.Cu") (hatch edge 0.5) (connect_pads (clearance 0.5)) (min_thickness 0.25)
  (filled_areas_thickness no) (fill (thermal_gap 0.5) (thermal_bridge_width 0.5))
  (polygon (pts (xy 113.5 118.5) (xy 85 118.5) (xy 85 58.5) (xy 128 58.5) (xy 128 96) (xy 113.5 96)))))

